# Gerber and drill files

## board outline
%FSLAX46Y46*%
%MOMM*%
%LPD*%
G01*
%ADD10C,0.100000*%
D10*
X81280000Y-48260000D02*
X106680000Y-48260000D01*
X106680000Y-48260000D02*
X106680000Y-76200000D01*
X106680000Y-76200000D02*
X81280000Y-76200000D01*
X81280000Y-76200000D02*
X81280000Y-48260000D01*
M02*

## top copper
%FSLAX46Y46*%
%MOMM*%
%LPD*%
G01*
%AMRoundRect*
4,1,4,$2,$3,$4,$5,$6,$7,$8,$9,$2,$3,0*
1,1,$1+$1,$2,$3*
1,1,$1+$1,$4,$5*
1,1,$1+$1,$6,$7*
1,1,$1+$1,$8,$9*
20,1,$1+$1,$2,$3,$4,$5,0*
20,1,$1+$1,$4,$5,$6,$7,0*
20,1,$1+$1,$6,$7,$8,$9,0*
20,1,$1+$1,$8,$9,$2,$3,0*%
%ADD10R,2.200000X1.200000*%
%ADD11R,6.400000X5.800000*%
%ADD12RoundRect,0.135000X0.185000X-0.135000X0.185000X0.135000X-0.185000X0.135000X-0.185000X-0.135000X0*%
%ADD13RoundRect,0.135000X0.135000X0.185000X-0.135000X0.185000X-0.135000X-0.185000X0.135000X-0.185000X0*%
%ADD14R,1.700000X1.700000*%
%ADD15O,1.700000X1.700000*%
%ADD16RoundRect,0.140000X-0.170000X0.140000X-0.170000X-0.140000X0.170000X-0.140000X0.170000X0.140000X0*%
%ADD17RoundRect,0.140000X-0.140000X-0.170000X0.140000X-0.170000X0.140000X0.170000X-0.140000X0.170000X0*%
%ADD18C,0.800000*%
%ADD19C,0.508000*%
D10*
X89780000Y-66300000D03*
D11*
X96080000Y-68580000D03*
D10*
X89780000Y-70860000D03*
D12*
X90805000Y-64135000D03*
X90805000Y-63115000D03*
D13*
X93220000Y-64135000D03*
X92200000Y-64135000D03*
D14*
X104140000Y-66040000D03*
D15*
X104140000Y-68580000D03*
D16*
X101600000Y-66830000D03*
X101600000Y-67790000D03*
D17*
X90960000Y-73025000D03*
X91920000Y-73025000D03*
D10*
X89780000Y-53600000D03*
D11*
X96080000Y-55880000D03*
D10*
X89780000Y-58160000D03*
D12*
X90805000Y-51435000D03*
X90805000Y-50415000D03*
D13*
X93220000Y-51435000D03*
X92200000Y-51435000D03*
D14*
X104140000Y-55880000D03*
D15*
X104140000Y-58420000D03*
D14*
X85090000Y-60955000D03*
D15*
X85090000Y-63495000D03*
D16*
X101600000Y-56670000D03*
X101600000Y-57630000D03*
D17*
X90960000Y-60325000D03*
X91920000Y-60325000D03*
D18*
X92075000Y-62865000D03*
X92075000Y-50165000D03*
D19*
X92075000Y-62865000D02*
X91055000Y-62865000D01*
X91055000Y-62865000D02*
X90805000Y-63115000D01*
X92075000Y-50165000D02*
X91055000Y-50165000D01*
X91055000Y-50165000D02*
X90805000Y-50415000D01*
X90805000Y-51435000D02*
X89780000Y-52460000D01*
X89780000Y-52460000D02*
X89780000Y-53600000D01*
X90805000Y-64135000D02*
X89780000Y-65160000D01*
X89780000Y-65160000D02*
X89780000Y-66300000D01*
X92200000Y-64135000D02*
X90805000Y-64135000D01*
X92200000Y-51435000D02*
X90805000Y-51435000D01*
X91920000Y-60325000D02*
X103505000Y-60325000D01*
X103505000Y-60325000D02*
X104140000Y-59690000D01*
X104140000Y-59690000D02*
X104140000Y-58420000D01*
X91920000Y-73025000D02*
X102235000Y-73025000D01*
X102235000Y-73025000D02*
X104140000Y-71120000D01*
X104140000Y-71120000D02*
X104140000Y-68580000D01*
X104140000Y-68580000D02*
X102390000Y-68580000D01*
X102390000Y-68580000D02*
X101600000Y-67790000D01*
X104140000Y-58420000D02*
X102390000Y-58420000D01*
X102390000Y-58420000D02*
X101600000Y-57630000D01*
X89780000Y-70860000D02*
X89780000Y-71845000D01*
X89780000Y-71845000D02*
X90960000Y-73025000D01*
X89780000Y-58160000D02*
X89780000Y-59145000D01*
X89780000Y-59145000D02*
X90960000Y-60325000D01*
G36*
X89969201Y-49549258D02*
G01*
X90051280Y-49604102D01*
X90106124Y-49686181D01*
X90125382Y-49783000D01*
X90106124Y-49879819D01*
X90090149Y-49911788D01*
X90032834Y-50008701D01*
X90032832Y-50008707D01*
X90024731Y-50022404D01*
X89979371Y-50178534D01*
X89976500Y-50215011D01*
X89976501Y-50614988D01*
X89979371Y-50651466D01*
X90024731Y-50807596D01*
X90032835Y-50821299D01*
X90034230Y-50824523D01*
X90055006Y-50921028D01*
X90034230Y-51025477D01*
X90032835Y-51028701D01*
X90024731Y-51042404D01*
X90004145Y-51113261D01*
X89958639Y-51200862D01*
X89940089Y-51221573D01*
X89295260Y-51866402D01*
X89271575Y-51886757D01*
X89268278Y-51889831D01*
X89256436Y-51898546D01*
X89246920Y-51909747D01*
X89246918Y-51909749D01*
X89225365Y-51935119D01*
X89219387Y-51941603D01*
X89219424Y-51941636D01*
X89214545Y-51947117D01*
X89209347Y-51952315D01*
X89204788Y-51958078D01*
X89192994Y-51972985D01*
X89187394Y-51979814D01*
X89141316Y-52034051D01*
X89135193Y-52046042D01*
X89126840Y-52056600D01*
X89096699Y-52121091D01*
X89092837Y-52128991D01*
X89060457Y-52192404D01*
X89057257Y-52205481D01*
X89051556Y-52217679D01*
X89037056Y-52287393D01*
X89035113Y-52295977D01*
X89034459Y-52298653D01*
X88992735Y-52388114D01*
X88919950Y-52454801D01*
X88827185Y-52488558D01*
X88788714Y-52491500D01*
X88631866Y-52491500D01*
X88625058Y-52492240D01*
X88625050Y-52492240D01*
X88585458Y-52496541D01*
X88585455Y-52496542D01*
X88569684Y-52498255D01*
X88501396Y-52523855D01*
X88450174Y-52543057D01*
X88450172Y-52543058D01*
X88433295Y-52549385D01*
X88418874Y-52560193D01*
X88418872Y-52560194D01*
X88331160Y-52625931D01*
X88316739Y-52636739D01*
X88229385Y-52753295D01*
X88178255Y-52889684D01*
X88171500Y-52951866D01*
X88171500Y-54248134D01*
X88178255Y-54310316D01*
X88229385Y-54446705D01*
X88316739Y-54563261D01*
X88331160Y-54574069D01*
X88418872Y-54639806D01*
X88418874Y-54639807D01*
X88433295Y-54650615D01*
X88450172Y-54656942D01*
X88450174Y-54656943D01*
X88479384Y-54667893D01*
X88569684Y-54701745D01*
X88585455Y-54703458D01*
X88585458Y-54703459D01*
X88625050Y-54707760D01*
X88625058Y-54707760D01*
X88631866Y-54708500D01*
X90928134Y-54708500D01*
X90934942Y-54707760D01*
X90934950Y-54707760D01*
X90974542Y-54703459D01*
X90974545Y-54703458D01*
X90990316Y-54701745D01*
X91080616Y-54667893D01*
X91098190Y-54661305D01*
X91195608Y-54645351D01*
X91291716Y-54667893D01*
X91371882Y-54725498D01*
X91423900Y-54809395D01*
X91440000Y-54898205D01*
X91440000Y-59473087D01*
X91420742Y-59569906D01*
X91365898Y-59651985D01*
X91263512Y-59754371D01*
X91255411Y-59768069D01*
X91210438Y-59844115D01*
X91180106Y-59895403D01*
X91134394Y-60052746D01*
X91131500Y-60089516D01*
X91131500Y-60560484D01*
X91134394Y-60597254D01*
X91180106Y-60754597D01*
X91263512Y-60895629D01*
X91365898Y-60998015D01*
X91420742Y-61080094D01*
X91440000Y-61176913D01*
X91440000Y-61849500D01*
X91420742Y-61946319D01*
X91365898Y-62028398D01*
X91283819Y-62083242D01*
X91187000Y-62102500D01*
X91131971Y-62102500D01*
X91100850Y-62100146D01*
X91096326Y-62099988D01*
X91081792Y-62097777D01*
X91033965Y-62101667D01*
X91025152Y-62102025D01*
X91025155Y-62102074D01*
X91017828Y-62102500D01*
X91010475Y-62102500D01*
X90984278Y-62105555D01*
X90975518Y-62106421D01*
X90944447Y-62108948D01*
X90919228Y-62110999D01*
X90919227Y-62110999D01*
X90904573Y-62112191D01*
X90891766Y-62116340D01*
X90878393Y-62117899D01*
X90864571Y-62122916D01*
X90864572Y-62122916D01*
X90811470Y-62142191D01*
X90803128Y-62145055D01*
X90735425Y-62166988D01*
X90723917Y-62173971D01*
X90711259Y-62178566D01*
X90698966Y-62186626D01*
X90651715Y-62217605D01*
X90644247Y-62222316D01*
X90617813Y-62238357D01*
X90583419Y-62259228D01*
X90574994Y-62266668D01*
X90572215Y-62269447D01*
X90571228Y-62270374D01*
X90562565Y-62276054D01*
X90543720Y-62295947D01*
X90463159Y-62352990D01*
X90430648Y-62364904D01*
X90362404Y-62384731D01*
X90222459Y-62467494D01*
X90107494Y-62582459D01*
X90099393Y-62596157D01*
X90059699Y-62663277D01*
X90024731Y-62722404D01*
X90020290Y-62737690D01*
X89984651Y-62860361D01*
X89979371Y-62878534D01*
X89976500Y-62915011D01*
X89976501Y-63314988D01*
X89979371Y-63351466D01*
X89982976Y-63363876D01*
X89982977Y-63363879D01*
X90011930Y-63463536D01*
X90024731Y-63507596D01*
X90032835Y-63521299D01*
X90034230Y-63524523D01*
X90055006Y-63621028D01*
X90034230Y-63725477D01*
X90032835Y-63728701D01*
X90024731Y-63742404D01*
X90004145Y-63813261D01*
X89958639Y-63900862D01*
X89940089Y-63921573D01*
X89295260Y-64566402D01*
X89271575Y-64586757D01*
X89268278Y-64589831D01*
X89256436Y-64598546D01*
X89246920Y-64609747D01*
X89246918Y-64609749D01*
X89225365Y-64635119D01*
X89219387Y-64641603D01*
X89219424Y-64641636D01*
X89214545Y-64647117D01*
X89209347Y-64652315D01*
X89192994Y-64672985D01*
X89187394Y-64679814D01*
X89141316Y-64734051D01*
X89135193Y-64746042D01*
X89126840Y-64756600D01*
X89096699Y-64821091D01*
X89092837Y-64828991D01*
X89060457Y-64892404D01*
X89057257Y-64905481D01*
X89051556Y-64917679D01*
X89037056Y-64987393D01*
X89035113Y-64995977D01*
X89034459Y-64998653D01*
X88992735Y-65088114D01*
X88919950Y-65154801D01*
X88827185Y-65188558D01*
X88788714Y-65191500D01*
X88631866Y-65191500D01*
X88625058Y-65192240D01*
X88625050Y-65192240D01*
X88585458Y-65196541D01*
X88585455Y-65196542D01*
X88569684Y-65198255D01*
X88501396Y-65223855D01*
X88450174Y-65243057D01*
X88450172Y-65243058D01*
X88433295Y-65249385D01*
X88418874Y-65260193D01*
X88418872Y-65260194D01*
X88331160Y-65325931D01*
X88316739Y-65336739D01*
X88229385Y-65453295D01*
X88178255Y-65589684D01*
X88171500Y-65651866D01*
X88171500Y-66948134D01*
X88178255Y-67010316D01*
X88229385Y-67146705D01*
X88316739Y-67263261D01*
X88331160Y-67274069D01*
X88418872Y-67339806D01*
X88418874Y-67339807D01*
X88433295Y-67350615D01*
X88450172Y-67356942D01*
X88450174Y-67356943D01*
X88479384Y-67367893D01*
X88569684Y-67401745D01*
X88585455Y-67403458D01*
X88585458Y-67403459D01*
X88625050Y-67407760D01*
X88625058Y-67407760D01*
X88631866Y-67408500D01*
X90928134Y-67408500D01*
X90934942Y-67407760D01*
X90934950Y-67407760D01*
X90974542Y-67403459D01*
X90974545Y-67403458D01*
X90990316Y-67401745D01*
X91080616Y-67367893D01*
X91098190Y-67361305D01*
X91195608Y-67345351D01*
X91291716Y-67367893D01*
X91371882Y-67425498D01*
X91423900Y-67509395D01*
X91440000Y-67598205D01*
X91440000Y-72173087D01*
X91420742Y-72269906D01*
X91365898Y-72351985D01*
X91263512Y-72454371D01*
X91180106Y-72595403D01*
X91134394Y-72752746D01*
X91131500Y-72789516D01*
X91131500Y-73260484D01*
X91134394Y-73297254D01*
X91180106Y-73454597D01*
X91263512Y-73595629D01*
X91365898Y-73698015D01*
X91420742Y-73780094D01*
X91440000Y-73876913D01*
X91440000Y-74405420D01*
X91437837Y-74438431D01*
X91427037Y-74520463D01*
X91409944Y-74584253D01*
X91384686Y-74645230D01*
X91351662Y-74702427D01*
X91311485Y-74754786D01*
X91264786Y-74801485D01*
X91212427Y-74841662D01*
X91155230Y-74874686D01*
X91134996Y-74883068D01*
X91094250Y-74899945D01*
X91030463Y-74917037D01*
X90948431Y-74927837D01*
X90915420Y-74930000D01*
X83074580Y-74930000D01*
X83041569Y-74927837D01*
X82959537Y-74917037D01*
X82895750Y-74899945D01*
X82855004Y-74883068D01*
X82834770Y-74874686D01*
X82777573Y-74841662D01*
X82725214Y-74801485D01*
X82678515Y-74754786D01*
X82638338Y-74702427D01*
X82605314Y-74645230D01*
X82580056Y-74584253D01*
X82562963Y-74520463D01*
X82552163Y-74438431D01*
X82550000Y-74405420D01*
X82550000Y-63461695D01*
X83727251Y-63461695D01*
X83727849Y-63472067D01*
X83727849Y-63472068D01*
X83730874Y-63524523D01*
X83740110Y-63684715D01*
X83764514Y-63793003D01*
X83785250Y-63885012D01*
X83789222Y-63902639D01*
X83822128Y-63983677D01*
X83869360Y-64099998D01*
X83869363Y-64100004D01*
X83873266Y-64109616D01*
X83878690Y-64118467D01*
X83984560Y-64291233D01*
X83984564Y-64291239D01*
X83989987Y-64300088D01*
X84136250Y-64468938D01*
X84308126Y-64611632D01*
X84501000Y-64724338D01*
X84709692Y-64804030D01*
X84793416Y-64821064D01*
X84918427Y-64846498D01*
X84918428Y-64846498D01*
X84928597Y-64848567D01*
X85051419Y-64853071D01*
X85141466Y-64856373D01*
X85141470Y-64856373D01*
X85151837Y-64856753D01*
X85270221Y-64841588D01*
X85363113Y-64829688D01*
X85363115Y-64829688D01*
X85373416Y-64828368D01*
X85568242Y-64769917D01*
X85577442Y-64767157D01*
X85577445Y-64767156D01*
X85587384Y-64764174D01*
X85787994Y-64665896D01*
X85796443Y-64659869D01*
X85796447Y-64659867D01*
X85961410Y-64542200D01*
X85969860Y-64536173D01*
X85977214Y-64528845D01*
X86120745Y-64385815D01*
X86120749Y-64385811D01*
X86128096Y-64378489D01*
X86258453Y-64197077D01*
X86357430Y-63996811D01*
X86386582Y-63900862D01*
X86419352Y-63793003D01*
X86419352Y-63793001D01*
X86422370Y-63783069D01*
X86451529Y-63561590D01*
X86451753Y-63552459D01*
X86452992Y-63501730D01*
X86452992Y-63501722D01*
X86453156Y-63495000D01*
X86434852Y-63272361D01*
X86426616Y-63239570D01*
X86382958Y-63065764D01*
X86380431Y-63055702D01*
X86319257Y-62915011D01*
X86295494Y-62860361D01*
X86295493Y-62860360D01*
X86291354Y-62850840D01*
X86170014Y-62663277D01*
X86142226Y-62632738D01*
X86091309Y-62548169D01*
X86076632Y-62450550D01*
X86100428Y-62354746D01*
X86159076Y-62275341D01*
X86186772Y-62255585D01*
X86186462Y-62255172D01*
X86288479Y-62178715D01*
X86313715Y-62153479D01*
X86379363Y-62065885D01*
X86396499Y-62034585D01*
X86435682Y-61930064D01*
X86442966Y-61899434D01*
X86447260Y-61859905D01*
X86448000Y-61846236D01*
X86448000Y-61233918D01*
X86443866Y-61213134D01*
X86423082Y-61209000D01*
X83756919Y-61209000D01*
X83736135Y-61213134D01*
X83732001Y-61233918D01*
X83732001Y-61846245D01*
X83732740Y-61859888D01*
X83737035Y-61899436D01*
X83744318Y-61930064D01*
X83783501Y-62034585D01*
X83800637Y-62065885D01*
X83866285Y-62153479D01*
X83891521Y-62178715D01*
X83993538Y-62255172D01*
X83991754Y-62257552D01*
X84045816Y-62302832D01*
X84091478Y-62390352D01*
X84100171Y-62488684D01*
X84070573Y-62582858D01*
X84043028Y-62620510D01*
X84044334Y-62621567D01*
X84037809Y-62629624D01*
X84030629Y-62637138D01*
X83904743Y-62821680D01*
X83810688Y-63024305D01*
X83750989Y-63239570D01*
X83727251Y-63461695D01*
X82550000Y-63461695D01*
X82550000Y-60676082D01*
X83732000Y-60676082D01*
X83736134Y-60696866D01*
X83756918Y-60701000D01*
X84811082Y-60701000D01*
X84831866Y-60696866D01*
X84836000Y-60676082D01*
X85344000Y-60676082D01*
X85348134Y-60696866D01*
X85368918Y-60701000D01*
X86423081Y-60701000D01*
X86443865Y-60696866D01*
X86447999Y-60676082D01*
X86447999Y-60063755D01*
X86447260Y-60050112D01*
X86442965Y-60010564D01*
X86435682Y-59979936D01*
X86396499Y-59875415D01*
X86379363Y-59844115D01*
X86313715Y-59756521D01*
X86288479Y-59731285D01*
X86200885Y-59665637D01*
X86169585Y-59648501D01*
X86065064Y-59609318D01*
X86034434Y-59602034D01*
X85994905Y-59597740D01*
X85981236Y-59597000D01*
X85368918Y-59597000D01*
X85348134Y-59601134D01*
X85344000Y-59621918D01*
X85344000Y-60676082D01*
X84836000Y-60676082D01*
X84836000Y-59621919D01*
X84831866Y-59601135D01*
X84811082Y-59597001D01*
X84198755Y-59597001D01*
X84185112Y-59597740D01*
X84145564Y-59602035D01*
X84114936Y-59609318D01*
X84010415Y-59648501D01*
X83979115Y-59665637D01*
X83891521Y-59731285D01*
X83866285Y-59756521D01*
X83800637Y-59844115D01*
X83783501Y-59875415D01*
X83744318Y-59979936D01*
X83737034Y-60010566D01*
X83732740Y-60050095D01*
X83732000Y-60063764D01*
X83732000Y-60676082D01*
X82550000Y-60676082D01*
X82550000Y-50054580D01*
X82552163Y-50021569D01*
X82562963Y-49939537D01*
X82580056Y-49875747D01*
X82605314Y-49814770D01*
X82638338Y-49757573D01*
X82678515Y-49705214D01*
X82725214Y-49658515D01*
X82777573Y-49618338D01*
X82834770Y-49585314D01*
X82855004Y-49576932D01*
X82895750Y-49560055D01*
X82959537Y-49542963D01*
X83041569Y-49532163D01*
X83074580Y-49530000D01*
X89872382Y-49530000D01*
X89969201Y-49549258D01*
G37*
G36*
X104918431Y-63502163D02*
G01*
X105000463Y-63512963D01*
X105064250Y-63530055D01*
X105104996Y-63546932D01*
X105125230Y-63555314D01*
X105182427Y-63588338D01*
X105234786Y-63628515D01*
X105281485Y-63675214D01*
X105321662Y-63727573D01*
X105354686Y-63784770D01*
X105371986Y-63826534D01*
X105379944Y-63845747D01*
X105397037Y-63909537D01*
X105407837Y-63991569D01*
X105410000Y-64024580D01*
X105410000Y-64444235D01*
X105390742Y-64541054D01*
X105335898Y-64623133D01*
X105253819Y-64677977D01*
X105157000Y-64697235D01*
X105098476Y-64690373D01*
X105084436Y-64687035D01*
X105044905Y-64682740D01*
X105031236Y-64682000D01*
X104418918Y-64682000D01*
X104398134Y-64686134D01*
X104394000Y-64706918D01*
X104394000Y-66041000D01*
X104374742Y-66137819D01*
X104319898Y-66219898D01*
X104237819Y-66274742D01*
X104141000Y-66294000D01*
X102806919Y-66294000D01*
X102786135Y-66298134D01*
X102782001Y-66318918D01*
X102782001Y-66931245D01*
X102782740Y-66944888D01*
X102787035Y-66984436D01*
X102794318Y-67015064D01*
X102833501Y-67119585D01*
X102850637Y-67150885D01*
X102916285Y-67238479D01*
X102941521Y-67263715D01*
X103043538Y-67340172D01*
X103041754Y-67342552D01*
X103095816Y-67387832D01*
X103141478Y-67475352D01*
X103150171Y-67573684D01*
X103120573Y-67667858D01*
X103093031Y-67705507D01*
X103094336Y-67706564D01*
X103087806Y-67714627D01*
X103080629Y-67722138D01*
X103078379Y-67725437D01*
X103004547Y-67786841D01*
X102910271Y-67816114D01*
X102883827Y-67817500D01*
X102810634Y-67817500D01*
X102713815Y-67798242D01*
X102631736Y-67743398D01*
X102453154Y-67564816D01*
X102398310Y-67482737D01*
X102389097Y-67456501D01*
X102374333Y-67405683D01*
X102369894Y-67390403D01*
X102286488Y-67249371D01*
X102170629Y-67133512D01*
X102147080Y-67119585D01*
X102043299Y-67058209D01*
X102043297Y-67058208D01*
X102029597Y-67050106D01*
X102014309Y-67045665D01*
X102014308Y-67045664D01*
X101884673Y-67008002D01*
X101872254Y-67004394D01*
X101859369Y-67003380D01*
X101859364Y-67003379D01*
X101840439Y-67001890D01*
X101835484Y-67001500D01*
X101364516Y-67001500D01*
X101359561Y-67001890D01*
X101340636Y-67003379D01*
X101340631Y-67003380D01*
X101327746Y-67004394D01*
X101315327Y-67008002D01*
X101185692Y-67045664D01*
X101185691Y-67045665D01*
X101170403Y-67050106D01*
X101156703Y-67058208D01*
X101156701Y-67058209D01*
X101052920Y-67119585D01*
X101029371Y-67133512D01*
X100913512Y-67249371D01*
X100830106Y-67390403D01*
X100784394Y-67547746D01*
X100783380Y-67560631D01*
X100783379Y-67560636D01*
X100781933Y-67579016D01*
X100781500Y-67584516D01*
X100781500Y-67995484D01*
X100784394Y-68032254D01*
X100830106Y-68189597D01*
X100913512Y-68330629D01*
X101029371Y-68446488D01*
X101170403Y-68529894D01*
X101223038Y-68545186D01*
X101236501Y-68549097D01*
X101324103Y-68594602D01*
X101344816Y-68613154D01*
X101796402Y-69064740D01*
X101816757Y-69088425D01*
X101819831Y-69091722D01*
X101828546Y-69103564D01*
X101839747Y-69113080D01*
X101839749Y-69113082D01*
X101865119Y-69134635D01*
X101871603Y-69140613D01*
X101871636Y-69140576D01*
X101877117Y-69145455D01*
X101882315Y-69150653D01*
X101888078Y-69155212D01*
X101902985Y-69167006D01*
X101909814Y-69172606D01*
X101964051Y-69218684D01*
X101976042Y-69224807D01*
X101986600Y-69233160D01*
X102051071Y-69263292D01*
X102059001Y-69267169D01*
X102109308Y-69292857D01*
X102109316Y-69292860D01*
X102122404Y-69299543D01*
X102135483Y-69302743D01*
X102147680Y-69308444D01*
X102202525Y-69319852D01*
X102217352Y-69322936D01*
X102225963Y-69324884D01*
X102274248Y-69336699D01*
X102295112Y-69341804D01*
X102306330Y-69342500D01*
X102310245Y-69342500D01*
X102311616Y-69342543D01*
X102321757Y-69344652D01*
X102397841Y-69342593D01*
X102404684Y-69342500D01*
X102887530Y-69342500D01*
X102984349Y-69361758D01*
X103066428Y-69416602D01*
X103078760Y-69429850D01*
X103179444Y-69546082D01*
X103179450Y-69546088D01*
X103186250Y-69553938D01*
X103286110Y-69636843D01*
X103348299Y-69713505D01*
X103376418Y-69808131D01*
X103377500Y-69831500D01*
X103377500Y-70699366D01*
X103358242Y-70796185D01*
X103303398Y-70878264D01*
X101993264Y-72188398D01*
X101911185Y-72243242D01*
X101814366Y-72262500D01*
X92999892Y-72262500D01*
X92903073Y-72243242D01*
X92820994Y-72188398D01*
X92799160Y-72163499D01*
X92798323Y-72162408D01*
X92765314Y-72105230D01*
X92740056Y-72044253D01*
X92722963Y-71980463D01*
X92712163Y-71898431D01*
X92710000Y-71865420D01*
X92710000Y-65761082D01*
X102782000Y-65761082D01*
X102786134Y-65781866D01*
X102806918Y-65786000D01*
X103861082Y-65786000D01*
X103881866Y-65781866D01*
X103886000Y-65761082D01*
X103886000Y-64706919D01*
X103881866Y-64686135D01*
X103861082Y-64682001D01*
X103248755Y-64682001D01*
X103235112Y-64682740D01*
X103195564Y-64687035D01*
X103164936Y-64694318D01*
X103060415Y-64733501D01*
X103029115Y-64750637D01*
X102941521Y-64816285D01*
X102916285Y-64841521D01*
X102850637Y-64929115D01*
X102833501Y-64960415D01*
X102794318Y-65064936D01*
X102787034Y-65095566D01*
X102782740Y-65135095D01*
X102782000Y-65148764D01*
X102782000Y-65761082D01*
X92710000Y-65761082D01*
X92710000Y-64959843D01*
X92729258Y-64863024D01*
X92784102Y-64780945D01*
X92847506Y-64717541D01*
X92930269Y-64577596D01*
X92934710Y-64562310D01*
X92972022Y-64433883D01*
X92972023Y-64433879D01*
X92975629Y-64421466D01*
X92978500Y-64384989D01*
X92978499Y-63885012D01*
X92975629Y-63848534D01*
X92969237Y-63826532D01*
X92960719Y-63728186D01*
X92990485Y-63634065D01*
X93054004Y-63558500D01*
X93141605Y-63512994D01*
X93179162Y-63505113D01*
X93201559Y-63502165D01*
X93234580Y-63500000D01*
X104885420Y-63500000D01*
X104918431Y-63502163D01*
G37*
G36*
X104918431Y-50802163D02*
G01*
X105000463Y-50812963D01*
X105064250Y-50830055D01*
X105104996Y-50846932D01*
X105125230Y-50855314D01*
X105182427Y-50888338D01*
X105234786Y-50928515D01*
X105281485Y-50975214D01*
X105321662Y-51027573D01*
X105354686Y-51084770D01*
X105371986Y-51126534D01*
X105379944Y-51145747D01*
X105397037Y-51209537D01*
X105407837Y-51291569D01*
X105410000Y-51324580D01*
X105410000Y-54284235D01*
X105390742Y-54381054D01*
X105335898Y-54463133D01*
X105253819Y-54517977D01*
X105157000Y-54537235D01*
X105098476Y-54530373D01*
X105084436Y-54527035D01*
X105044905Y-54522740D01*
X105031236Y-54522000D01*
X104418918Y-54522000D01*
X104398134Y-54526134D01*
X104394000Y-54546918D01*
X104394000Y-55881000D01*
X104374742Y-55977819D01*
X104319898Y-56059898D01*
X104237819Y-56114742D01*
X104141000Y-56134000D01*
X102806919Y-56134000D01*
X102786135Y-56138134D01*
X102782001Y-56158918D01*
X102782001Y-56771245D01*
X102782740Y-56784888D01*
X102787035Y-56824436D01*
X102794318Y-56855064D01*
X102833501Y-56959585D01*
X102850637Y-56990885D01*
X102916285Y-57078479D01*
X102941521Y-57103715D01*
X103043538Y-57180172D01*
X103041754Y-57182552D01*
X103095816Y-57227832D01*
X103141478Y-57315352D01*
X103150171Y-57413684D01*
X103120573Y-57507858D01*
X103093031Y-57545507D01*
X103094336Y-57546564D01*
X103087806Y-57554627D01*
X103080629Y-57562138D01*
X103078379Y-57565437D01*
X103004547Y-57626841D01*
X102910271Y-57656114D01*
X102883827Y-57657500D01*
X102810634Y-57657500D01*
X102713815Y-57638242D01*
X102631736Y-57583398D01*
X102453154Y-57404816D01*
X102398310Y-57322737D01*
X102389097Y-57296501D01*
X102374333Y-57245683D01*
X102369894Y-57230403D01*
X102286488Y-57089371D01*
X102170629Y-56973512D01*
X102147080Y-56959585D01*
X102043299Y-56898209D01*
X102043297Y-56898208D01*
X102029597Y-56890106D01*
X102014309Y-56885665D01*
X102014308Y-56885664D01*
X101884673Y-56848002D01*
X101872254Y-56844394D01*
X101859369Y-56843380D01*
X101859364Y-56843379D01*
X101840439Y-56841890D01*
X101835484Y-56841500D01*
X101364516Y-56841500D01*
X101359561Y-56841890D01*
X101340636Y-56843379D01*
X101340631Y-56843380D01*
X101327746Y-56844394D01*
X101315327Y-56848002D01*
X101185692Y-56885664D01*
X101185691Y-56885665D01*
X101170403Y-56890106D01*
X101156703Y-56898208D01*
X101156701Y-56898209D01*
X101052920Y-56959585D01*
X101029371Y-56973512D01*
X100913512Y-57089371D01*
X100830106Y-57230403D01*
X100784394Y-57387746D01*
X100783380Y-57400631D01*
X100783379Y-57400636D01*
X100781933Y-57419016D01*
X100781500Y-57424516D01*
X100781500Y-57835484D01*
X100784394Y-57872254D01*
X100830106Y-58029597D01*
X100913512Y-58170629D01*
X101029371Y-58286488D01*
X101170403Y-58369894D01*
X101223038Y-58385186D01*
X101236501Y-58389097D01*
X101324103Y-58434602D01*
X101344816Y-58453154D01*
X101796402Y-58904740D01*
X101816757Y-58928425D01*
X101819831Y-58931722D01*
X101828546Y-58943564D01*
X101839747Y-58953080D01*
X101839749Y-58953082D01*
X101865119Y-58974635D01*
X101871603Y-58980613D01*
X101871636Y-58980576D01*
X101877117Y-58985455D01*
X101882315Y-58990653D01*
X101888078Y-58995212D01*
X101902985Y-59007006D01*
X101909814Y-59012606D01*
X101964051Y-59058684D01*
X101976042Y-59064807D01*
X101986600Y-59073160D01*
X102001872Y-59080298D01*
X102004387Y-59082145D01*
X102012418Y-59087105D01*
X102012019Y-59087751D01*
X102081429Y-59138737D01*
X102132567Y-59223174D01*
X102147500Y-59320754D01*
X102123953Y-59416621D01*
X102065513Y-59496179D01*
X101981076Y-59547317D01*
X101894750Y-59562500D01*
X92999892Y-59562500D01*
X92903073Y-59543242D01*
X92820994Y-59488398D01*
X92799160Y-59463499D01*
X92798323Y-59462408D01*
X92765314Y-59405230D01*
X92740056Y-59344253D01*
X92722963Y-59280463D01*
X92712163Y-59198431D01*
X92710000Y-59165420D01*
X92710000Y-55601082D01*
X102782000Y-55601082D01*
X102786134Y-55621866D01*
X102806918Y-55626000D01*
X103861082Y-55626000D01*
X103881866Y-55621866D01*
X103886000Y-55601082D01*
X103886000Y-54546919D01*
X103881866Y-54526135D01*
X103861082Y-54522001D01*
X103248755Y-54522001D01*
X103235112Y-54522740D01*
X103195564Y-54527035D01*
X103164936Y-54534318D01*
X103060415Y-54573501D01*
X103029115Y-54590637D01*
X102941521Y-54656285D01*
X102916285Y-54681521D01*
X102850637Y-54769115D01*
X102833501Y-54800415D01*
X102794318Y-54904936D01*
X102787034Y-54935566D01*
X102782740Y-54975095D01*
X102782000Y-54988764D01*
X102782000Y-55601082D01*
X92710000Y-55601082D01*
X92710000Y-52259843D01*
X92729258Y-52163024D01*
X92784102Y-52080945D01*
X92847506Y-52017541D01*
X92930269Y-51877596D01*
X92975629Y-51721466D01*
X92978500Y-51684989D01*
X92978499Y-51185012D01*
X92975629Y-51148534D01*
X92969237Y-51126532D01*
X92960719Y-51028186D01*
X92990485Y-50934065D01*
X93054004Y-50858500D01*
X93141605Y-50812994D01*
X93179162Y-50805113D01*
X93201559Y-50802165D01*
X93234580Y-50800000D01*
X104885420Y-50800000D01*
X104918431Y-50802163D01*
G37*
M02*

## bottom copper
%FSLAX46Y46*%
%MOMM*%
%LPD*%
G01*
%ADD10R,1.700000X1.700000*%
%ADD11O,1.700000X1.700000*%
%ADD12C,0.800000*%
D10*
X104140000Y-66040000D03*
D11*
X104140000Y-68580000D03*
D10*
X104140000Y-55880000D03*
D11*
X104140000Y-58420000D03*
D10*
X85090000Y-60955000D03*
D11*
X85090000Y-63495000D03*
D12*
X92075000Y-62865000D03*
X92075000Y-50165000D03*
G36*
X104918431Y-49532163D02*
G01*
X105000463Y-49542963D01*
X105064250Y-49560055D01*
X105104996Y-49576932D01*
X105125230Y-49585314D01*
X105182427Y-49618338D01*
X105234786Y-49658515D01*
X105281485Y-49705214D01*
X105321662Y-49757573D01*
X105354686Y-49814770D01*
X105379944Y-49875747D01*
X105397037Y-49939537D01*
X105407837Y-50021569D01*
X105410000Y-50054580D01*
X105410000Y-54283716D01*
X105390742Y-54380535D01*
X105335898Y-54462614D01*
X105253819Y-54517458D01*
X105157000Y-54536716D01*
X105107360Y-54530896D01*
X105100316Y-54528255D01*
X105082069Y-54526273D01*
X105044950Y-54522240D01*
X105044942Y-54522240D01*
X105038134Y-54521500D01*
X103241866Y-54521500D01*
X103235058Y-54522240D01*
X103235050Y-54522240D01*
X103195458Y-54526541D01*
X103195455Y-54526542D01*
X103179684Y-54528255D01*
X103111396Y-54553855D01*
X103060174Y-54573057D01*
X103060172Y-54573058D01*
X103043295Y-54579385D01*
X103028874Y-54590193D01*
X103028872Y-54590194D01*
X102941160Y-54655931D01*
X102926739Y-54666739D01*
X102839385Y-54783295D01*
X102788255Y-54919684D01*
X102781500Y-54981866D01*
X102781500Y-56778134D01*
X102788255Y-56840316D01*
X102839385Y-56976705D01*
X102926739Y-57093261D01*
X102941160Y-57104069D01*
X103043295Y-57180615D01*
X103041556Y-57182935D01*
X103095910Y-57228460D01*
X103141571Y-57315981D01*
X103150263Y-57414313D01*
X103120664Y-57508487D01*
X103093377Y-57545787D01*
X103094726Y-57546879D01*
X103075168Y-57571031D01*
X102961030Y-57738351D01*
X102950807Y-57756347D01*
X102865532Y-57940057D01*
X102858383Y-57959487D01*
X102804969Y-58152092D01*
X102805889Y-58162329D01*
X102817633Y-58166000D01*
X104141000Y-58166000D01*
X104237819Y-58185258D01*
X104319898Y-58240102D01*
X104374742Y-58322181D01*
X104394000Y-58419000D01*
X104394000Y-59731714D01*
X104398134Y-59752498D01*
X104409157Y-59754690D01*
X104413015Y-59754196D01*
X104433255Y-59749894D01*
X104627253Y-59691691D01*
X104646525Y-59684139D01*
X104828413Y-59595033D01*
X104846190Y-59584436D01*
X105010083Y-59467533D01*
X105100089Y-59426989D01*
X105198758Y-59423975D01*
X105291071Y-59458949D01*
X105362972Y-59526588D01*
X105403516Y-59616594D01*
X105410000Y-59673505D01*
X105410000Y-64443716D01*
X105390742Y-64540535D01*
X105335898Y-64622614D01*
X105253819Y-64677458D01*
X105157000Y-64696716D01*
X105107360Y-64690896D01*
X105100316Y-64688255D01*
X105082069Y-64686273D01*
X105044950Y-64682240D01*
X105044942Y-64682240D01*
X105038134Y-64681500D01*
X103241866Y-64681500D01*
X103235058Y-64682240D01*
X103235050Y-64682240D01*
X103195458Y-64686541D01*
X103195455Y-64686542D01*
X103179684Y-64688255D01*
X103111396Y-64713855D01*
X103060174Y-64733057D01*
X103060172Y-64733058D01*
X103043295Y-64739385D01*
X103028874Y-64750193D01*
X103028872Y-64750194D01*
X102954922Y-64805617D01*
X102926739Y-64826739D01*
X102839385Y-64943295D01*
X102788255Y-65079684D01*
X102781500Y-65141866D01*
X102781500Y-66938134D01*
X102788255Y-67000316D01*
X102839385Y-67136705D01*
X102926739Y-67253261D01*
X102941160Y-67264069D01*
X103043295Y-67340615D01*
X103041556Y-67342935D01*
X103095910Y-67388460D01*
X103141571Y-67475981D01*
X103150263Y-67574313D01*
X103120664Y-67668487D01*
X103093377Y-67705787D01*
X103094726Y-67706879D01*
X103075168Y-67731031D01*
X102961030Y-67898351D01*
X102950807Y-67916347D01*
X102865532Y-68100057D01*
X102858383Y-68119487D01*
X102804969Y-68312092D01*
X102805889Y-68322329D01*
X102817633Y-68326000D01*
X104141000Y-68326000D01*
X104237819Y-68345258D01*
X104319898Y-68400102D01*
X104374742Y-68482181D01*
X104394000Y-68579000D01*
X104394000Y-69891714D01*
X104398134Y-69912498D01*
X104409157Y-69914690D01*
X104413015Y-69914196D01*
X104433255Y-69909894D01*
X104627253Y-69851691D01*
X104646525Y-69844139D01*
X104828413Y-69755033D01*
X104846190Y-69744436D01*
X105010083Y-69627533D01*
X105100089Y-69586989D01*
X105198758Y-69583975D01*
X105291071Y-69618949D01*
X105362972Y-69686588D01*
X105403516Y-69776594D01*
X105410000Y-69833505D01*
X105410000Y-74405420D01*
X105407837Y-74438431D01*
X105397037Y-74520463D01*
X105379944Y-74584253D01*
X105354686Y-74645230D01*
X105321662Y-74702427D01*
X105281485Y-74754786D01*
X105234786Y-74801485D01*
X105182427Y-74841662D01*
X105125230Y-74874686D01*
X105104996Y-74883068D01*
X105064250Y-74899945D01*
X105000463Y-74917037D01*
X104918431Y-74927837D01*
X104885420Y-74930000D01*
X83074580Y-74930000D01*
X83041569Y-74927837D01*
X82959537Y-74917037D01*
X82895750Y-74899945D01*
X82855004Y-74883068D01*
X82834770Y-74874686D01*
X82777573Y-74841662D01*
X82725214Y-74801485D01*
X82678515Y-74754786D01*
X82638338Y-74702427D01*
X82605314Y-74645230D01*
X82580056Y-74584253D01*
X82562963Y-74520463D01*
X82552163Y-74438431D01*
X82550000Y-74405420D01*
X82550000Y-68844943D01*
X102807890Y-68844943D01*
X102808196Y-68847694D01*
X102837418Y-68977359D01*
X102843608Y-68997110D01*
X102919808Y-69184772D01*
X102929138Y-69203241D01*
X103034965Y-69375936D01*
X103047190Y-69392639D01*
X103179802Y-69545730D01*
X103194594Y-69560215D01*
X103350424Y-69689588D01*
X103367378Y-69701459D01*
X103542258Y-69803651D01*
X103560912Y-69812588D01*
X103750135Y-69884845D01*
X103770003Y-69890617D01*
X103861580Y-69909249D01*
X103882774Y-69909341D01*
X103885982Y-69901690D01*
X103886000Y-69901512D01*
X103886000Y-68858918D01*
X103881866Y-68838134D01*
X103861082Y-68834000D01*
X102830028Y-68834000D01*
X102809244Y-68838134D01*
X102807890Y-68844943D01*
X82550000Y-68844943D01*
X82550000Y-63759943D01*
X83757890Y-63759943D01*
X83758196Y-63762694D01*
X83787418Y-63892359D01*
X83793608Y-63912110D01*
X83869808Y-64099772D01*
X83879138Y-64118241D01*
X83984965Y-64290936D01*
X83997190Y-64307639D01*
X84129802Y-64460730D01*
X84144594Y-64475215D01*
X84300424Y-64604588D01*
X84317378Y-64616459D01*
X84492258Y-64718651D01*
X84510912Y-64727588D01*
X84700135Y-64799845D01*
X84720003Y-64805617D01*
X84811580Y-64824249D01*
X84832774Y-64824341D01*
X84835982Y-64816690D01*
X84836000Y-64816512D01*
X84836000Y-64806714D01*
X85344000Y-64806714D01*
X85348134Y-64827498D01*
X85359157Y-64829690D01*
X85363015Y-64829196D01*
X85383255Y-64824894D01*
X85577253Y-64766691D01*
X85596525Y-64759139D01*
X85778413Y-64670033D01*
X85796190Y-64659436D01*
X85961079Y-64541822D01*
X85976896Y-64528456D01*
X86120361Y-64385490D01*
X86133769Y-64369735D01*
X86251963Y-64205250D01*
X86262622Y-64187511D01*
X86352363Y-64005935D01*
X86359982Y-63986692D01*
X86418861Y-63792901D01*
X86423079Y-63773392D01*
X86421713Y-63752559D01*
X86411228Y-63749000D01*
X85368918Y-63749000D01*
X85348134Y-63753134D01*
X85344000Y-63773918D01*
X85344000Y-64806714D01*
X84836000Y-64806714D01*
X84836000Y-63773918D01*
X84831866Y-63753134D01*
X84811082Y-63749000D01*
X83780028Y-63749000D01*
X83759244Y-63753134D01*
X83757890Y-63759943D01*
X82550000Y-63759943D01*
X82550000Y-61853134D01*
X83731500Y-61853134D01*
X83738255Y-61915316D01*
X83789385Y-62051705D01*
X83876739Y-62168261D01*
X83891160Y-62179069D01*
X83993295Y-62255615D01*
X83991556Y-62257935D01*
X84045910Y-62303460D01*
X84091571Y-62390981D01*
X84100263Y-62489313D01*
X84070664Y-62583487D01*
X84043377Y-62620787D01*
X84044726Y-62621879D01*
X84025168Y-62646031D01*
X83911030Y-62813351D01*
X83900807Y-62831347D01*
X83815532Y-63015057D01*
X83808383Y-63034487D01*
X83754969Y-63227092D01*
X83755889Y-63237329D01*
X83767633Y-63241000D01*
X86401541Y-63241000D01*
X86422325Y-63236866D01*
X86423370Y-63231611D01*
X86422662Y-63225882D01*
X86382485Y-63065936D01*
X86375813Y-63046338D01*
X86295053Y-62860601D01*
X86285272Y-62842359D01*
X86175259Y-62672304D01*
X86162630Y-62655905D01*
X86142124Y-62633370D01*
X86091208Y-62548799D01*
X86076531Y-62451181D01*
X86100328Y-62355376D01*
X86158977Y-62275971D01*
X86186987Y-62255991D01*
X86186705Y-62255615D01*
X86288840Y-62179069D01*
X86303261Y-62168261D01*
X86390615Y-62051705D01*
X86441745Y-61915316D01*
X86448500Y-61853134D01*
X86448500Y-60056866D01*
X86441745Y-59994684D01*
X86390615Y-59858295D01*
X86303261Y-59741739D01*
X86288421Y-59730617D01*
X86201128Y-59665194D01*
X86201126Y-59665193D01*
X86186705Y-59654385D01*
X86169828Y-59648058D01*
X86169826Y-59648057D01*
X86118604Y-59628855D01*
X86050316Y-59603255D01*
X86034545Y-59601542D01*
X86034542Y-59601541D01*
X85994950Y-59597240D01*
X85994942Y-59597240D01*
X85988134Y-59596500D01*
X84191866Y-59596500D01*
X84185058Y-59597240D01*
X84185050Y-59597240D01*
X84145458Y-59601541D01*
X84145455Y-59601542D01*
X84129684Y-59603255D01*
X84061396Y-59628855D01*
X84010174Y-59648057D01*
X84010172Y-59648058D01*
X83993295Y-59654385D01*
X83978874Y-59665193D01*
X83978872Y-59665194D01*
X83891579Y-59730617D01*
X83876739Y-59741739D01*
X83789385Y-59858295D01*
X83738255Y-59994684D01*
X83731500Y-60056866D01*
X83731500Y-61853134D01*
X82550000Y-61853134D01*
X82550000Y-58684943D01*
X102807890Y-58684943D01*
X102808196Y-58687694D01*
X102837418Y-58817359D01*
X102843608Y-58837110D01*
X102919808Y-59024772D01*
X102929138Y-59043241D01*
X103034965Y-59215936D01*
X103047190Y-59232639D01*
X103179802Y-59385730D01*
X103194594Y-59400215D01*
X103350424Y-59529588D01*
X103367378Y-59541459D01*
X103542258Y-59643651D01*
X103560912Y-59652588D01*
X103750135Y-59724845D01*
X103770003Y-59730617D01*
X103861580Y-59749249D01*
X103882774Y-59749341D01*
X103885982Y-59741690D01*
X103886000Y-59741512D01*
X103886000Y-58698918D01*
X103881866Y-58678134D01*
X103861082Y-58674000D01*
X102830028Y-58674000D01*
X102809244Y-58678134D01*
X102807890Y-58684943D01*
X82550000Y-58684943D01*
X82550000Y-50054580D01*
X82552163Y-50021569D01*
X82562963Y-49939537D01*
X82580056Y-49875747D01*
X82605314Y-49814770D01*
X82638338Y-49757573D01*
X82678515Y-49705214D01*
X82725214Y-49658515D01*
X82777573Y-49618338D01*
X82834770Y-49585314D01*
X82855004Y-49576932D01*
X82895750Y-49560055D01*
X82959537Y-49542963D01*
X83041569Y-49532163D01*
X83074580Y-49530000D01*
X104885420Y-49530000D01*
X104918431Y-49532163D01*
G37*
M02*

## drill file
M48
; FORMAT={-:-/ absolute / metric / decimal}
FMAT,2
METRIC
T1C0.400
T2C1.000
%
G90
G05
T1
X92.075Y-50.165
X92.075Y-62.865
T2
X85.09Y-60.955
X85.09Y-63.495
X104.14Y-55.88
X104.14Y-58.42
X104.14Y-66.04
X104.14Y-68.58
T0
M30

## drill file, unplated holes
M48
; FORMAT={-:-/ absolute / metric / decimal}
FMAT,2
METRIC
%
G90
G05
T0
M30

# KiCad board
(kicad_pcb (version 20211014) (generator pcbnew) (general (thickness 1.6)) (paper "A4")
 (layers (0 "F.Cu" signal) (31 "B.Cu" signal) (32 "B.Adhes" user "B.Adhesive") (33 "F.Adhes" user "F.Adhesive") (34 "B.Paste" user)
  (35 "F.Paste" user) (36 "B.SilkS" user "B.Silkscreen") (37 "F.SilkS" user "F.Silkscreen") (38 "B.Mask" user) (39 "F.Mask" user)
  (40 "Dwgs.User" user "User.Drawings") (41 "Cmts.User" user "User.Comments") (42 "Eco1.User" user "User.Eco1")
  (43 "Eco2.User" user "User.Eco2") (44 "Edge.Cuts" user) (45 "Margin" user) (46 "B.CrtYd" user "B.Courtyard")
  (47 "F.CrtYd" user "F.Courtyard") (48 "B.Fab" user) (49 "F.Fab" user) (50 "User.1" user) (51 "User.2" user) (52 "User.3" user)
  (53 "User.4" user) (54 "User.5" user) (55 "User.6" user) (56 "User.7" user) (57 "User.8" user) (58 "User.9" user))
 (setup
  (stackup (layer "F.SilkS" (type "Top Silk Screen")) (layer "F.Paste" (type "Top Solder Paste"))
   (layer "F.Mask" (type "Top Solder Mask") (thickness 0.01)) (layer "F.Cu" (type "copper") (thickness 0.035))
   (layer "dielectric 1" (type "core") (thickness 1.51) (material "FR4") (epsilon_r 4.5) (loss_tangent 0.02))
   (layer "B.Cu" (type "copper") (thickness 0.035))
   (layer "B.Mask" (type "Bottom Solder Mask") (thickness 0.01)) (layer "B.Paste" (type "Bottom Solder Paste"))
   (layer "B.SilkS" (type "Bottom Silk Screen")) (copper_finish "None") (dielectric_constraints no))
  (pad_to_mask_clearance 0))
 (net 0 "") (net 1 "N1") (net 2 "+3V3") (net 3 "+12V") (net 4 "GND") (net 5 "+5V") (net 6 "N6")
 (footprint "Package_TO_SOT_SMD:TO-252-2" (layer "F.Cu") (at 93.98 68.58)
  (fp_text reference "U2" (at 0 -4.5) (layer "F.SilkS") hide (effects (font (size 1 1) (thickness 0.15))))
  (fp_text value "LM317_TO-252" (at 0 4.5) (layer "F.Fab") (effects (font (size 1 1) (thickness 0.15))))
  (pad "" smd rect (at 3.775 1.525) (size 3.05 2.75) (layers "F.Paste"))
  (pad "" smd rect (at 0.425 1.525) (size 3.05 2.75) (layers "F.Paste"))
  (pad "" smd rect (at 0.425 -1.525) (size 3.05 2.75) (layers "F.Paste"))
  (pad "" smd rect (at 3.775 -1.525) (size 3.05 2.75) (layers "F.Paste"))
  (pad "1" smd rect (at -4.2 -2.28) (size 2.2 1.2) (layers "F.Cu" "F.Paste" "F.Mask") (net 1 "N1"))
  (pad "2" smd rect (at 2.1 0) (size 6.4 5.8) (layers "F.Cu" "F.Mask") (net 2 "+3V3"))
  (pad "3" smd rect (at -4.2 2.28) (size 2.2 1.2) (layers "F.Cu" "F.Paste" "F.Mask") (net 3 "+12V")))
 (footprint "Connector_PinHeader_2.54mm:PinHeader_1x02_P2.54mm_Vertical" (layer "F.Cu") (at 104.14 66.04)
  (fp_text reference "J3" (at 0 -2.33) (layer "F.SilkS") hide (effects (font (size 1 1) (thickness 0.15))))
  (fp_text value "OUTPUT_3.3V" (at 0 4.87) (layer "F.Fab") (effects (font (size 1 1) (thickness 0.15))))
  (pad "1" thru_hole rect (at 0 0) (size 1.7 1.7) (drill 1) (layers *.Cu *.Mask) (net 2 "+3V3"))
  (pad "2" thru_hole oval (at 0 2.54) (size 1.7 1.7) (drill 1) (layers *.Cu *.Mask) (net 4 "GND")))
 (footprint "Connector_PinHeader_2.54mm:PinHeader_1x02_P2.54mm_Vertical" (layer "F.Cu") (at 104.14 55.88)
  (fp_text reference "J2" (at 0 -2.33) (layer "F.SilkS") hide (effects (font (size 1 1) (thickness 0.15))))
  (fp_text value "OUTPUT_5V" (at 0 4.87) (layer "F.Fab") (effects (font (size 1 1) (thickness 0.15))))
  (pad "1" thru_hole rect (at 0 0) (size 1.7 1.7) (drill 1) (layers *.Cu *.Mask) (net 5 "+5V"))
  (pad "2" thru_hole oval (at 0 2.54) (size 1.7 1.7) (drill 1) (layers *.Cu *.Mask) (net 4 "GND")))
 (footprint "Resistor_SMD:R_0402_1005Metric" (layer "F.Cu") (at 92.71 64.135 180)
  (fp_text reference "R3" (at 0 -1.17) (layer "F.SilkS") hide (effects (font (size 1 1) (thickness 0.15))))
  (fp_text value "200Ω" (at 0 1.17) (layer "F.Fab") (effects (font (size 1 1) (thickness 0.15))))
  (pad "1" smd roundrect (at -0.51 0 180) (size 0.54 0.64) (layers "F.Cu" "F.Paste" "F.Mask") (roundrect_rratio 0.25) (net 2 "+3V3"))
  (pad "2" smd roundrect (at 0.51 0 180) (size 0.54 0.64) (layers "F.Cu" "F.Paste" "F.Mask") (roundrect_rratio 0.25) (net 1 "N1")))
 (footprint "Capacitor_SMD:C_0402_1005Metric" (layer "F.Cu") (at 91.44 60.325)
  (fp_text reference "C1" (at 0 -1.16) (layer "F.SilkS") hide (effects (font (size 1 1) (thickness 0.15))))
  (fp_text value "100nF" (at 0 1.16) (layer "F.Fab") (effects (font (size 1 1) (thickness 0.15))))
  (pad "1" smd roundrect (at -0.48 0) (size 0.56 0.62) (layers "F.Cu" "F.Paste" "F.Mask") (roundrect_rratio 0.25) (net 3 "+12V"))
  (pad "2" smd roundrect (at 0.48 0) (size 0.56 0.62) (layers "F.Cu" "F.Paste" "F.Mask") (roundrect_rratio 0.25) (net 4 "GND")))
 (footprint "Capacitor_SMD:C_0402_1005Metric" (layer "F.Cu") (at 91.44 73.025)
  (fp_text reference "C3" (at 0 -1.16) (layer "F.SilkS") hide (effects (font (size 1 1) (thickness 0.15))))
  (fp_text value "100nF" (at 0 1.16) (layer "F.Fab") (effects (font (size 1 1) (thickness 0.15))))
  (pad "1" smd roundrect (at -0.48 0) (size 0.56 0.62) (layers "F.Cu" "F.Paste" "F.Mask") (roundrect_rratio 0.25) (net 3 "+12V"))
  (pad "2" smd roundrect (at 0.48 0) (size 0.56 0.62) (layers "F.Cu" "F.Paste" "F.Mask") (roundrect_rratio 0.25) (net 4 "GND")))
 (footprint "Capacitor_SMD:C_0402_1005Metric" (layer "F.Cu") (at 101.6 67.31 -90)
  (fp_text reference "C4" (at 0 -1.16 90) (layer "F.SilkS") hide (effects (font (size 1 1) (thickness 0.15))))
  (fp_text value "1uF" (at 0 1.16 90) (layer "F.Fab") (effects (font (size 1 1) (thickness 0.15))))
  (pad "1" smd roundrect (at -0.48 0 270) (size 0.56 0.62) (layers "F.Cu" "F.Paste" "F.Mask") (roundrect_rratio 0.25) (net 2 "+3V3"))
  (pad "2" smd roundrect (at 0.48 0 270) (size 0.56 0.62) (layers "F.Cu" "F.Paste" "F.Mask") (roundrect_rratio 0.25) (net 4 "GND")))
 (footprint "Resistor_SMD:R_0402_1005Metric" (layer "F.Cu") (at 90.805 50.925 90)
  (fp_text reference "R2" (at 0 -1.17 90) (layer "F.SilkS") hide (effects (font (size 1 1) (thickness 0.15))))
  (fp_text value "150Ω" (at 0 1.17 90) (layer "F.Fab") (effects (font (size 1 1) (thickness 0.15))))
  (pad "1" smd roundrect (at -0.51 0 90) (size 0.54 0.64) (layers "F.Cu" "F.Paste" "F.Mask") (roundrect_rratio 0.25) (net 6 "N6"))
  (pad "2" smd roundrect (at 0.51 0 90) (size 0.54 0.64) (layers "F.Cu" "F.Paste" "F.Mask") (roundrect_rratio 0.25) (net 4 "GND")))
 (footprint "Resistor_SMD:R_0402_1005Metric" (layer "F.Cu") (at 90.805 63.625 90)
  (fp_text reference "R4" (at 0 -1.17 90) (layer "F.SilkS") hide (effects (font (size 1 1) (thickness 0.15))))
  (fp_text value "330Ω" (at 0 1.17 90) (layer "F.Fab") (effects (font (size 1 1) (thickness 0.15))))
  (pad "1" smd roundrect (at -0.51 0 90) (size 0.54 0.64) (layers "F.Cu" "F.Paste" "F.Mask") (roundrect_rratio 0.25) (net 1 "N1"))
  (pad "2" smd roundrect (at 0.51 0 90) (size 0.54 0.64) (layers "F.Cu" "F.Paste" "F.Mask") (roundrect_rratio 0.25) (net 4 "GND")))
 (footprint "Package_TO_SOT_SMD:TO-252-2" (layer "F.Cu") (at 93.98 55.88)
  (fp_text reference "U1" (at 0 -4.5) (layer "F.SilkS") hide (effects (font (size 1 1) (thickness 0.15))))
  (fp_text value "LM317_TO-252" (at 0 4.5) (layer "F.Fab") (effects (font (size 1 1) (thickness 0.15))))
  (pad "" smd rect (at 3.775 -1.525) (size 3.05 2.75) (layers "F.Paste"))
  (pad "" smd rect (at 0.425 1.525) (size 3.05 2.75) (layers "F.Paste"))
  (pad "" smd rect (at 0.425 -1.525) (size 3.05 2.75) (layers "F.Paste"))
  (pad "" smd rect (at 3.775 1.525) (size 3.05 2.75) (layers "F.Paste"))
  (pad "1" smd rect (at -4.2 -2.28) (size 2.2 1.2) (layers "F.Cu" "F.Paste" "F.Mask") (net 6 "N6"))
  (pad "2" smd rect (at 2.1 0) (size 6.4 5.8) (layers "F.Cu" "F.Mask") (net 5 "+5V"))
  (pad "3" smd rect (at -4.2 2.28) (size 2.2 1.2) (layers "F.Cu" "F.Paste" "F.Mask") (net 3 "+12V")))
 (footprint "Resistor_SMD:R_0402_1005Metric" (layer "F.Cu") (at 92.71 51.435 180)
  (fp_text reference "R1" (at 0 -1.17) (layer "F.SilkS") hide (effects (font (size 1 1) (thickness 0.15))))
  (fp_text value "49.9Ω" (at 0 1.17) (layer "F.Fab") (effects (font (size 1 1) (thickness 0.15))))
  (pad "1" smd roundrect (at -0.51 0 180) (size 0.54 0.64) (layers "F.Cu" "F.Paste" "F.Mask") (roundrect_rratio 0.25) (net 5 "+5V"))
  (pad "2" smd roundrect (at 0.51 0 180) (size 0.54 0.64) (layers "F.Cu" "F.Paste" "F.Mask") (roundrect_rratio 0.25) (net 6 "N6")))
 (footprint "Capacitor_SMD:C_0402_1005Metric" (layer "F.Cu") (at 101.6 57.15 -90)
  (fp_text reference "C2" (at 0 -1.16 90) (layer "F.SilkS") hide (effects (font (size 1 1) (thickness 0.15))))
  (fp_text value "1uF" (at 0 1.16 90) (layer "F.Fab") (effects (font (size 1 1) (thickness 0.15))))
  (pad "1" smd roundrect (at -0.48 0 270) (size 0.56 0.62) (layers "F.Cu" "F.Paste" "F.Mask") (roundrect_rratio 0.25) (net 5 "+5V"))
  (pad "2" smd roundrect (at 0.48 0 270) (size 0.56 0.62) (layers "F.Cu" "F.Paste" "F.Mask") (roundrect_rratio 0.25) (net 4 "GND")))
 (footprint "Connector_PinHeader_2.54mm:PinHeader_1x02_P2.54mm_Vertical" (layer "F.Cu") (at 85.09 60.955)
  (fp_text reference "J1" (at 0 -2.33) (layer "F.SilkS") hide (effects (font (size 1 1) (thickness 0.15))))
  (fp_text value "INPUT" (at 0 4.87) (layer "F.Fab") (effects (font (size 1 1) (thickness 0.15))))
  (pad "1" thru_hole rect (at 0 0) (size 1.7 1.7) (drill 1) (layers *.Cu *.Mask) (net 3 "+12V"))
  (pad "2" thru_hole oval (at 0 2.54) (size 1.7 1.7) (drill 1) (layers *.Cu *.Mask) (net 4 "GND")))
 (gr_rect (start 81.28 48.26) (end 106.68 76.2) (layer "Edge.Cuts") (width 0.1) (fill none))
 (segment (start 89.78 71.845) (end 90.96 73.025) (width 0.508) (layer "F.Cu") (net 3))
 (segment (start 89.78 58.16) (end 89.78 59.145) (width 0.508) (layer "F.Cu") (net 3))
 (segment (start 89.78 59.145) (end 90.96 60.325) (width 0.508) (layer "F.Cu") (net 3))
 (segment (start 89.78 70.86) (end 89.78 71.845) (width 0.508) (layer "F.Cu") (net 3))
 (segment (start 92.075 50.165) (end 91.055 50.165) (width 0.508) (layer "F.Cu") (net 4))
 (segment (start 91.92 73.025) (end 102.235 73.025) (width 0.508) (layer "F.Cu") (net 4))
 (segment (start 104.14 58.42) (end 102.39 58.42) (width 0.508) (layer "F.Cu") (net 4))
 (segment (start 102.39 58.42) (end 101.6 57.63) (width 0.508) (layer "F.Cu") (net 4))
 (segment (start 103.505 60.325) (end 104.14 59.69) (width 0.508) (layer "F.Cu") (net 4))
 (segment (start 104.14 68.58) (end 102.39 68.58) (width 0.508) (layer "F.Cu") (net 4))
 (segment (start 104.14 71.12) (end 104.14 68.58) (width 0.508) (layer "F.Cu") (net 4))
 (segment (start 91.055 50.165) (end 90.805 50.415) (width 0.508) (layer "F.Cu") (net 4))
 (segment (start 91.055 62.865) (end 90.805 63.115) (width 0.508) (layer "F.Cu") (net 4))
 (segment (start 102.39 68.58) (end 101.6 67.79) (width 0.508) (layer "F.Cu") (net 4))
 (segment (start 91.92 60.325) (end 103.505 60.325) (width 0.508) (layer "F.Cu") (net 4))
 (segment (start 92.075 62.865) (end 91.055 62.865) (width 0.508) (layer "F.Cu") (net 4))
 (segment (start 104.14 59.69) (end 104.14 58.42) (width 0.508) (layer "F.Cu") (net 4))
 (segment (start 102.235 73.025) (end 104.14 71.12) (width 0.508) (layer "F.Cu") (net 4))
 (via (at 92.075 62.865) (size 0.8) (drill 0.4) (layers "F.Cu" "B.Cu") (free) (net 4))
 (via (at 92.075 50.165) (size 0.8) (drill 0.4) (layers "F.Cu" "B.Cu") (free) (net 4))
 (segment (start 92.2 51.435) (end 90.805 51.435) (width 0.508) (layer "F.Cu") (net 6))
 (segment (start 90.805 51.435) (end 89.78 52.46) (width 0.508) (layer "F.Cu") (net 6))
 (segment (start 89.78 52.46) (end 89.78 53.6) (width 0.508) (layer "F.Cu") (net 6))
 (segment (start 90.805 64.135) (end 89.78 65.16) (width 0.508) (layer "F.Cu") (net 1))
 (segment (start 92.2 64.135) (end 90.805 64.135) (width 0.508) (layer "F.Cu") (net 1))
 (segment (start 89.78 65.16) (end 89.78 66.3) (width 0.508) (layer "F.Cu") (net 1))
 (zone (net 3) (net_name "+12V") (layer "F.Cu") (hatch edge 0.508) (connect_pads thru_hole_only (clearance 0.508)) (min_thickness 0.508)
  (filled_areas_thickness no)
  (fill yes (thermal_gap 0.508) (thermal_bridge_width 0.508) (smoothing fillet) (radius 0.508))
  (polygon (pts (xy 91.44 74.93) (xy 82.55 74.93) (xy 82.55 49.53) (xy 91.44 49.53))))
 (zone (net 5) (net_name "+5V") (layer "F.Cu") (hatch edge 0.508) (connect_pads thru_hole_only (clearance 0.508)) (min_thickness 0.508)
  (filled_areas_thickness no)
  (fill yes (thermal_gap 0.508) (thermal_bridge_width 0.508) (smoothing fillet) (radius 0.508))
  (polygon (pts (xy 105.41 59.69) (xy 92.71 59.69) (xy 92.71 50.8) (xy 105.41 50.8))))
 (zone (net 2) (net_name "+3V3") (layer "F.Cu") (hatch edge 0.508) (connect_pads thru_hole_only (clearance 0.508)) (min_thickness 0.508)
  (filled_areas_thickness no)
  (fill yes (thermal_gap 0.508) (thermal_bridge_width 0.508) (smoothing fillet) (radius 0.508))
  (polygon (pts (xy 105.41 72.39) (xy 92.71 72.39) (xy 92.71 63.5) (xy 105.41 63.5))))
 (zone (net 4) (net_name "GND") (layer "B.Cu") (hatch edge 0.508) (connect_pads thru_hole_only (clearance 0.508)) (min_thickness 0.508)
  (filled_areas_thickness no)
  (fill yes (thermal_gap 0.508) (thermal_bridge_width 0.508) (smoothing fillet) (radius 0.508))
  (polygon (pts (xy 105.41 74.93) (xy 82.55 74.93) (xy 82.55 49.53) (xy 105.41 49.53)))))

